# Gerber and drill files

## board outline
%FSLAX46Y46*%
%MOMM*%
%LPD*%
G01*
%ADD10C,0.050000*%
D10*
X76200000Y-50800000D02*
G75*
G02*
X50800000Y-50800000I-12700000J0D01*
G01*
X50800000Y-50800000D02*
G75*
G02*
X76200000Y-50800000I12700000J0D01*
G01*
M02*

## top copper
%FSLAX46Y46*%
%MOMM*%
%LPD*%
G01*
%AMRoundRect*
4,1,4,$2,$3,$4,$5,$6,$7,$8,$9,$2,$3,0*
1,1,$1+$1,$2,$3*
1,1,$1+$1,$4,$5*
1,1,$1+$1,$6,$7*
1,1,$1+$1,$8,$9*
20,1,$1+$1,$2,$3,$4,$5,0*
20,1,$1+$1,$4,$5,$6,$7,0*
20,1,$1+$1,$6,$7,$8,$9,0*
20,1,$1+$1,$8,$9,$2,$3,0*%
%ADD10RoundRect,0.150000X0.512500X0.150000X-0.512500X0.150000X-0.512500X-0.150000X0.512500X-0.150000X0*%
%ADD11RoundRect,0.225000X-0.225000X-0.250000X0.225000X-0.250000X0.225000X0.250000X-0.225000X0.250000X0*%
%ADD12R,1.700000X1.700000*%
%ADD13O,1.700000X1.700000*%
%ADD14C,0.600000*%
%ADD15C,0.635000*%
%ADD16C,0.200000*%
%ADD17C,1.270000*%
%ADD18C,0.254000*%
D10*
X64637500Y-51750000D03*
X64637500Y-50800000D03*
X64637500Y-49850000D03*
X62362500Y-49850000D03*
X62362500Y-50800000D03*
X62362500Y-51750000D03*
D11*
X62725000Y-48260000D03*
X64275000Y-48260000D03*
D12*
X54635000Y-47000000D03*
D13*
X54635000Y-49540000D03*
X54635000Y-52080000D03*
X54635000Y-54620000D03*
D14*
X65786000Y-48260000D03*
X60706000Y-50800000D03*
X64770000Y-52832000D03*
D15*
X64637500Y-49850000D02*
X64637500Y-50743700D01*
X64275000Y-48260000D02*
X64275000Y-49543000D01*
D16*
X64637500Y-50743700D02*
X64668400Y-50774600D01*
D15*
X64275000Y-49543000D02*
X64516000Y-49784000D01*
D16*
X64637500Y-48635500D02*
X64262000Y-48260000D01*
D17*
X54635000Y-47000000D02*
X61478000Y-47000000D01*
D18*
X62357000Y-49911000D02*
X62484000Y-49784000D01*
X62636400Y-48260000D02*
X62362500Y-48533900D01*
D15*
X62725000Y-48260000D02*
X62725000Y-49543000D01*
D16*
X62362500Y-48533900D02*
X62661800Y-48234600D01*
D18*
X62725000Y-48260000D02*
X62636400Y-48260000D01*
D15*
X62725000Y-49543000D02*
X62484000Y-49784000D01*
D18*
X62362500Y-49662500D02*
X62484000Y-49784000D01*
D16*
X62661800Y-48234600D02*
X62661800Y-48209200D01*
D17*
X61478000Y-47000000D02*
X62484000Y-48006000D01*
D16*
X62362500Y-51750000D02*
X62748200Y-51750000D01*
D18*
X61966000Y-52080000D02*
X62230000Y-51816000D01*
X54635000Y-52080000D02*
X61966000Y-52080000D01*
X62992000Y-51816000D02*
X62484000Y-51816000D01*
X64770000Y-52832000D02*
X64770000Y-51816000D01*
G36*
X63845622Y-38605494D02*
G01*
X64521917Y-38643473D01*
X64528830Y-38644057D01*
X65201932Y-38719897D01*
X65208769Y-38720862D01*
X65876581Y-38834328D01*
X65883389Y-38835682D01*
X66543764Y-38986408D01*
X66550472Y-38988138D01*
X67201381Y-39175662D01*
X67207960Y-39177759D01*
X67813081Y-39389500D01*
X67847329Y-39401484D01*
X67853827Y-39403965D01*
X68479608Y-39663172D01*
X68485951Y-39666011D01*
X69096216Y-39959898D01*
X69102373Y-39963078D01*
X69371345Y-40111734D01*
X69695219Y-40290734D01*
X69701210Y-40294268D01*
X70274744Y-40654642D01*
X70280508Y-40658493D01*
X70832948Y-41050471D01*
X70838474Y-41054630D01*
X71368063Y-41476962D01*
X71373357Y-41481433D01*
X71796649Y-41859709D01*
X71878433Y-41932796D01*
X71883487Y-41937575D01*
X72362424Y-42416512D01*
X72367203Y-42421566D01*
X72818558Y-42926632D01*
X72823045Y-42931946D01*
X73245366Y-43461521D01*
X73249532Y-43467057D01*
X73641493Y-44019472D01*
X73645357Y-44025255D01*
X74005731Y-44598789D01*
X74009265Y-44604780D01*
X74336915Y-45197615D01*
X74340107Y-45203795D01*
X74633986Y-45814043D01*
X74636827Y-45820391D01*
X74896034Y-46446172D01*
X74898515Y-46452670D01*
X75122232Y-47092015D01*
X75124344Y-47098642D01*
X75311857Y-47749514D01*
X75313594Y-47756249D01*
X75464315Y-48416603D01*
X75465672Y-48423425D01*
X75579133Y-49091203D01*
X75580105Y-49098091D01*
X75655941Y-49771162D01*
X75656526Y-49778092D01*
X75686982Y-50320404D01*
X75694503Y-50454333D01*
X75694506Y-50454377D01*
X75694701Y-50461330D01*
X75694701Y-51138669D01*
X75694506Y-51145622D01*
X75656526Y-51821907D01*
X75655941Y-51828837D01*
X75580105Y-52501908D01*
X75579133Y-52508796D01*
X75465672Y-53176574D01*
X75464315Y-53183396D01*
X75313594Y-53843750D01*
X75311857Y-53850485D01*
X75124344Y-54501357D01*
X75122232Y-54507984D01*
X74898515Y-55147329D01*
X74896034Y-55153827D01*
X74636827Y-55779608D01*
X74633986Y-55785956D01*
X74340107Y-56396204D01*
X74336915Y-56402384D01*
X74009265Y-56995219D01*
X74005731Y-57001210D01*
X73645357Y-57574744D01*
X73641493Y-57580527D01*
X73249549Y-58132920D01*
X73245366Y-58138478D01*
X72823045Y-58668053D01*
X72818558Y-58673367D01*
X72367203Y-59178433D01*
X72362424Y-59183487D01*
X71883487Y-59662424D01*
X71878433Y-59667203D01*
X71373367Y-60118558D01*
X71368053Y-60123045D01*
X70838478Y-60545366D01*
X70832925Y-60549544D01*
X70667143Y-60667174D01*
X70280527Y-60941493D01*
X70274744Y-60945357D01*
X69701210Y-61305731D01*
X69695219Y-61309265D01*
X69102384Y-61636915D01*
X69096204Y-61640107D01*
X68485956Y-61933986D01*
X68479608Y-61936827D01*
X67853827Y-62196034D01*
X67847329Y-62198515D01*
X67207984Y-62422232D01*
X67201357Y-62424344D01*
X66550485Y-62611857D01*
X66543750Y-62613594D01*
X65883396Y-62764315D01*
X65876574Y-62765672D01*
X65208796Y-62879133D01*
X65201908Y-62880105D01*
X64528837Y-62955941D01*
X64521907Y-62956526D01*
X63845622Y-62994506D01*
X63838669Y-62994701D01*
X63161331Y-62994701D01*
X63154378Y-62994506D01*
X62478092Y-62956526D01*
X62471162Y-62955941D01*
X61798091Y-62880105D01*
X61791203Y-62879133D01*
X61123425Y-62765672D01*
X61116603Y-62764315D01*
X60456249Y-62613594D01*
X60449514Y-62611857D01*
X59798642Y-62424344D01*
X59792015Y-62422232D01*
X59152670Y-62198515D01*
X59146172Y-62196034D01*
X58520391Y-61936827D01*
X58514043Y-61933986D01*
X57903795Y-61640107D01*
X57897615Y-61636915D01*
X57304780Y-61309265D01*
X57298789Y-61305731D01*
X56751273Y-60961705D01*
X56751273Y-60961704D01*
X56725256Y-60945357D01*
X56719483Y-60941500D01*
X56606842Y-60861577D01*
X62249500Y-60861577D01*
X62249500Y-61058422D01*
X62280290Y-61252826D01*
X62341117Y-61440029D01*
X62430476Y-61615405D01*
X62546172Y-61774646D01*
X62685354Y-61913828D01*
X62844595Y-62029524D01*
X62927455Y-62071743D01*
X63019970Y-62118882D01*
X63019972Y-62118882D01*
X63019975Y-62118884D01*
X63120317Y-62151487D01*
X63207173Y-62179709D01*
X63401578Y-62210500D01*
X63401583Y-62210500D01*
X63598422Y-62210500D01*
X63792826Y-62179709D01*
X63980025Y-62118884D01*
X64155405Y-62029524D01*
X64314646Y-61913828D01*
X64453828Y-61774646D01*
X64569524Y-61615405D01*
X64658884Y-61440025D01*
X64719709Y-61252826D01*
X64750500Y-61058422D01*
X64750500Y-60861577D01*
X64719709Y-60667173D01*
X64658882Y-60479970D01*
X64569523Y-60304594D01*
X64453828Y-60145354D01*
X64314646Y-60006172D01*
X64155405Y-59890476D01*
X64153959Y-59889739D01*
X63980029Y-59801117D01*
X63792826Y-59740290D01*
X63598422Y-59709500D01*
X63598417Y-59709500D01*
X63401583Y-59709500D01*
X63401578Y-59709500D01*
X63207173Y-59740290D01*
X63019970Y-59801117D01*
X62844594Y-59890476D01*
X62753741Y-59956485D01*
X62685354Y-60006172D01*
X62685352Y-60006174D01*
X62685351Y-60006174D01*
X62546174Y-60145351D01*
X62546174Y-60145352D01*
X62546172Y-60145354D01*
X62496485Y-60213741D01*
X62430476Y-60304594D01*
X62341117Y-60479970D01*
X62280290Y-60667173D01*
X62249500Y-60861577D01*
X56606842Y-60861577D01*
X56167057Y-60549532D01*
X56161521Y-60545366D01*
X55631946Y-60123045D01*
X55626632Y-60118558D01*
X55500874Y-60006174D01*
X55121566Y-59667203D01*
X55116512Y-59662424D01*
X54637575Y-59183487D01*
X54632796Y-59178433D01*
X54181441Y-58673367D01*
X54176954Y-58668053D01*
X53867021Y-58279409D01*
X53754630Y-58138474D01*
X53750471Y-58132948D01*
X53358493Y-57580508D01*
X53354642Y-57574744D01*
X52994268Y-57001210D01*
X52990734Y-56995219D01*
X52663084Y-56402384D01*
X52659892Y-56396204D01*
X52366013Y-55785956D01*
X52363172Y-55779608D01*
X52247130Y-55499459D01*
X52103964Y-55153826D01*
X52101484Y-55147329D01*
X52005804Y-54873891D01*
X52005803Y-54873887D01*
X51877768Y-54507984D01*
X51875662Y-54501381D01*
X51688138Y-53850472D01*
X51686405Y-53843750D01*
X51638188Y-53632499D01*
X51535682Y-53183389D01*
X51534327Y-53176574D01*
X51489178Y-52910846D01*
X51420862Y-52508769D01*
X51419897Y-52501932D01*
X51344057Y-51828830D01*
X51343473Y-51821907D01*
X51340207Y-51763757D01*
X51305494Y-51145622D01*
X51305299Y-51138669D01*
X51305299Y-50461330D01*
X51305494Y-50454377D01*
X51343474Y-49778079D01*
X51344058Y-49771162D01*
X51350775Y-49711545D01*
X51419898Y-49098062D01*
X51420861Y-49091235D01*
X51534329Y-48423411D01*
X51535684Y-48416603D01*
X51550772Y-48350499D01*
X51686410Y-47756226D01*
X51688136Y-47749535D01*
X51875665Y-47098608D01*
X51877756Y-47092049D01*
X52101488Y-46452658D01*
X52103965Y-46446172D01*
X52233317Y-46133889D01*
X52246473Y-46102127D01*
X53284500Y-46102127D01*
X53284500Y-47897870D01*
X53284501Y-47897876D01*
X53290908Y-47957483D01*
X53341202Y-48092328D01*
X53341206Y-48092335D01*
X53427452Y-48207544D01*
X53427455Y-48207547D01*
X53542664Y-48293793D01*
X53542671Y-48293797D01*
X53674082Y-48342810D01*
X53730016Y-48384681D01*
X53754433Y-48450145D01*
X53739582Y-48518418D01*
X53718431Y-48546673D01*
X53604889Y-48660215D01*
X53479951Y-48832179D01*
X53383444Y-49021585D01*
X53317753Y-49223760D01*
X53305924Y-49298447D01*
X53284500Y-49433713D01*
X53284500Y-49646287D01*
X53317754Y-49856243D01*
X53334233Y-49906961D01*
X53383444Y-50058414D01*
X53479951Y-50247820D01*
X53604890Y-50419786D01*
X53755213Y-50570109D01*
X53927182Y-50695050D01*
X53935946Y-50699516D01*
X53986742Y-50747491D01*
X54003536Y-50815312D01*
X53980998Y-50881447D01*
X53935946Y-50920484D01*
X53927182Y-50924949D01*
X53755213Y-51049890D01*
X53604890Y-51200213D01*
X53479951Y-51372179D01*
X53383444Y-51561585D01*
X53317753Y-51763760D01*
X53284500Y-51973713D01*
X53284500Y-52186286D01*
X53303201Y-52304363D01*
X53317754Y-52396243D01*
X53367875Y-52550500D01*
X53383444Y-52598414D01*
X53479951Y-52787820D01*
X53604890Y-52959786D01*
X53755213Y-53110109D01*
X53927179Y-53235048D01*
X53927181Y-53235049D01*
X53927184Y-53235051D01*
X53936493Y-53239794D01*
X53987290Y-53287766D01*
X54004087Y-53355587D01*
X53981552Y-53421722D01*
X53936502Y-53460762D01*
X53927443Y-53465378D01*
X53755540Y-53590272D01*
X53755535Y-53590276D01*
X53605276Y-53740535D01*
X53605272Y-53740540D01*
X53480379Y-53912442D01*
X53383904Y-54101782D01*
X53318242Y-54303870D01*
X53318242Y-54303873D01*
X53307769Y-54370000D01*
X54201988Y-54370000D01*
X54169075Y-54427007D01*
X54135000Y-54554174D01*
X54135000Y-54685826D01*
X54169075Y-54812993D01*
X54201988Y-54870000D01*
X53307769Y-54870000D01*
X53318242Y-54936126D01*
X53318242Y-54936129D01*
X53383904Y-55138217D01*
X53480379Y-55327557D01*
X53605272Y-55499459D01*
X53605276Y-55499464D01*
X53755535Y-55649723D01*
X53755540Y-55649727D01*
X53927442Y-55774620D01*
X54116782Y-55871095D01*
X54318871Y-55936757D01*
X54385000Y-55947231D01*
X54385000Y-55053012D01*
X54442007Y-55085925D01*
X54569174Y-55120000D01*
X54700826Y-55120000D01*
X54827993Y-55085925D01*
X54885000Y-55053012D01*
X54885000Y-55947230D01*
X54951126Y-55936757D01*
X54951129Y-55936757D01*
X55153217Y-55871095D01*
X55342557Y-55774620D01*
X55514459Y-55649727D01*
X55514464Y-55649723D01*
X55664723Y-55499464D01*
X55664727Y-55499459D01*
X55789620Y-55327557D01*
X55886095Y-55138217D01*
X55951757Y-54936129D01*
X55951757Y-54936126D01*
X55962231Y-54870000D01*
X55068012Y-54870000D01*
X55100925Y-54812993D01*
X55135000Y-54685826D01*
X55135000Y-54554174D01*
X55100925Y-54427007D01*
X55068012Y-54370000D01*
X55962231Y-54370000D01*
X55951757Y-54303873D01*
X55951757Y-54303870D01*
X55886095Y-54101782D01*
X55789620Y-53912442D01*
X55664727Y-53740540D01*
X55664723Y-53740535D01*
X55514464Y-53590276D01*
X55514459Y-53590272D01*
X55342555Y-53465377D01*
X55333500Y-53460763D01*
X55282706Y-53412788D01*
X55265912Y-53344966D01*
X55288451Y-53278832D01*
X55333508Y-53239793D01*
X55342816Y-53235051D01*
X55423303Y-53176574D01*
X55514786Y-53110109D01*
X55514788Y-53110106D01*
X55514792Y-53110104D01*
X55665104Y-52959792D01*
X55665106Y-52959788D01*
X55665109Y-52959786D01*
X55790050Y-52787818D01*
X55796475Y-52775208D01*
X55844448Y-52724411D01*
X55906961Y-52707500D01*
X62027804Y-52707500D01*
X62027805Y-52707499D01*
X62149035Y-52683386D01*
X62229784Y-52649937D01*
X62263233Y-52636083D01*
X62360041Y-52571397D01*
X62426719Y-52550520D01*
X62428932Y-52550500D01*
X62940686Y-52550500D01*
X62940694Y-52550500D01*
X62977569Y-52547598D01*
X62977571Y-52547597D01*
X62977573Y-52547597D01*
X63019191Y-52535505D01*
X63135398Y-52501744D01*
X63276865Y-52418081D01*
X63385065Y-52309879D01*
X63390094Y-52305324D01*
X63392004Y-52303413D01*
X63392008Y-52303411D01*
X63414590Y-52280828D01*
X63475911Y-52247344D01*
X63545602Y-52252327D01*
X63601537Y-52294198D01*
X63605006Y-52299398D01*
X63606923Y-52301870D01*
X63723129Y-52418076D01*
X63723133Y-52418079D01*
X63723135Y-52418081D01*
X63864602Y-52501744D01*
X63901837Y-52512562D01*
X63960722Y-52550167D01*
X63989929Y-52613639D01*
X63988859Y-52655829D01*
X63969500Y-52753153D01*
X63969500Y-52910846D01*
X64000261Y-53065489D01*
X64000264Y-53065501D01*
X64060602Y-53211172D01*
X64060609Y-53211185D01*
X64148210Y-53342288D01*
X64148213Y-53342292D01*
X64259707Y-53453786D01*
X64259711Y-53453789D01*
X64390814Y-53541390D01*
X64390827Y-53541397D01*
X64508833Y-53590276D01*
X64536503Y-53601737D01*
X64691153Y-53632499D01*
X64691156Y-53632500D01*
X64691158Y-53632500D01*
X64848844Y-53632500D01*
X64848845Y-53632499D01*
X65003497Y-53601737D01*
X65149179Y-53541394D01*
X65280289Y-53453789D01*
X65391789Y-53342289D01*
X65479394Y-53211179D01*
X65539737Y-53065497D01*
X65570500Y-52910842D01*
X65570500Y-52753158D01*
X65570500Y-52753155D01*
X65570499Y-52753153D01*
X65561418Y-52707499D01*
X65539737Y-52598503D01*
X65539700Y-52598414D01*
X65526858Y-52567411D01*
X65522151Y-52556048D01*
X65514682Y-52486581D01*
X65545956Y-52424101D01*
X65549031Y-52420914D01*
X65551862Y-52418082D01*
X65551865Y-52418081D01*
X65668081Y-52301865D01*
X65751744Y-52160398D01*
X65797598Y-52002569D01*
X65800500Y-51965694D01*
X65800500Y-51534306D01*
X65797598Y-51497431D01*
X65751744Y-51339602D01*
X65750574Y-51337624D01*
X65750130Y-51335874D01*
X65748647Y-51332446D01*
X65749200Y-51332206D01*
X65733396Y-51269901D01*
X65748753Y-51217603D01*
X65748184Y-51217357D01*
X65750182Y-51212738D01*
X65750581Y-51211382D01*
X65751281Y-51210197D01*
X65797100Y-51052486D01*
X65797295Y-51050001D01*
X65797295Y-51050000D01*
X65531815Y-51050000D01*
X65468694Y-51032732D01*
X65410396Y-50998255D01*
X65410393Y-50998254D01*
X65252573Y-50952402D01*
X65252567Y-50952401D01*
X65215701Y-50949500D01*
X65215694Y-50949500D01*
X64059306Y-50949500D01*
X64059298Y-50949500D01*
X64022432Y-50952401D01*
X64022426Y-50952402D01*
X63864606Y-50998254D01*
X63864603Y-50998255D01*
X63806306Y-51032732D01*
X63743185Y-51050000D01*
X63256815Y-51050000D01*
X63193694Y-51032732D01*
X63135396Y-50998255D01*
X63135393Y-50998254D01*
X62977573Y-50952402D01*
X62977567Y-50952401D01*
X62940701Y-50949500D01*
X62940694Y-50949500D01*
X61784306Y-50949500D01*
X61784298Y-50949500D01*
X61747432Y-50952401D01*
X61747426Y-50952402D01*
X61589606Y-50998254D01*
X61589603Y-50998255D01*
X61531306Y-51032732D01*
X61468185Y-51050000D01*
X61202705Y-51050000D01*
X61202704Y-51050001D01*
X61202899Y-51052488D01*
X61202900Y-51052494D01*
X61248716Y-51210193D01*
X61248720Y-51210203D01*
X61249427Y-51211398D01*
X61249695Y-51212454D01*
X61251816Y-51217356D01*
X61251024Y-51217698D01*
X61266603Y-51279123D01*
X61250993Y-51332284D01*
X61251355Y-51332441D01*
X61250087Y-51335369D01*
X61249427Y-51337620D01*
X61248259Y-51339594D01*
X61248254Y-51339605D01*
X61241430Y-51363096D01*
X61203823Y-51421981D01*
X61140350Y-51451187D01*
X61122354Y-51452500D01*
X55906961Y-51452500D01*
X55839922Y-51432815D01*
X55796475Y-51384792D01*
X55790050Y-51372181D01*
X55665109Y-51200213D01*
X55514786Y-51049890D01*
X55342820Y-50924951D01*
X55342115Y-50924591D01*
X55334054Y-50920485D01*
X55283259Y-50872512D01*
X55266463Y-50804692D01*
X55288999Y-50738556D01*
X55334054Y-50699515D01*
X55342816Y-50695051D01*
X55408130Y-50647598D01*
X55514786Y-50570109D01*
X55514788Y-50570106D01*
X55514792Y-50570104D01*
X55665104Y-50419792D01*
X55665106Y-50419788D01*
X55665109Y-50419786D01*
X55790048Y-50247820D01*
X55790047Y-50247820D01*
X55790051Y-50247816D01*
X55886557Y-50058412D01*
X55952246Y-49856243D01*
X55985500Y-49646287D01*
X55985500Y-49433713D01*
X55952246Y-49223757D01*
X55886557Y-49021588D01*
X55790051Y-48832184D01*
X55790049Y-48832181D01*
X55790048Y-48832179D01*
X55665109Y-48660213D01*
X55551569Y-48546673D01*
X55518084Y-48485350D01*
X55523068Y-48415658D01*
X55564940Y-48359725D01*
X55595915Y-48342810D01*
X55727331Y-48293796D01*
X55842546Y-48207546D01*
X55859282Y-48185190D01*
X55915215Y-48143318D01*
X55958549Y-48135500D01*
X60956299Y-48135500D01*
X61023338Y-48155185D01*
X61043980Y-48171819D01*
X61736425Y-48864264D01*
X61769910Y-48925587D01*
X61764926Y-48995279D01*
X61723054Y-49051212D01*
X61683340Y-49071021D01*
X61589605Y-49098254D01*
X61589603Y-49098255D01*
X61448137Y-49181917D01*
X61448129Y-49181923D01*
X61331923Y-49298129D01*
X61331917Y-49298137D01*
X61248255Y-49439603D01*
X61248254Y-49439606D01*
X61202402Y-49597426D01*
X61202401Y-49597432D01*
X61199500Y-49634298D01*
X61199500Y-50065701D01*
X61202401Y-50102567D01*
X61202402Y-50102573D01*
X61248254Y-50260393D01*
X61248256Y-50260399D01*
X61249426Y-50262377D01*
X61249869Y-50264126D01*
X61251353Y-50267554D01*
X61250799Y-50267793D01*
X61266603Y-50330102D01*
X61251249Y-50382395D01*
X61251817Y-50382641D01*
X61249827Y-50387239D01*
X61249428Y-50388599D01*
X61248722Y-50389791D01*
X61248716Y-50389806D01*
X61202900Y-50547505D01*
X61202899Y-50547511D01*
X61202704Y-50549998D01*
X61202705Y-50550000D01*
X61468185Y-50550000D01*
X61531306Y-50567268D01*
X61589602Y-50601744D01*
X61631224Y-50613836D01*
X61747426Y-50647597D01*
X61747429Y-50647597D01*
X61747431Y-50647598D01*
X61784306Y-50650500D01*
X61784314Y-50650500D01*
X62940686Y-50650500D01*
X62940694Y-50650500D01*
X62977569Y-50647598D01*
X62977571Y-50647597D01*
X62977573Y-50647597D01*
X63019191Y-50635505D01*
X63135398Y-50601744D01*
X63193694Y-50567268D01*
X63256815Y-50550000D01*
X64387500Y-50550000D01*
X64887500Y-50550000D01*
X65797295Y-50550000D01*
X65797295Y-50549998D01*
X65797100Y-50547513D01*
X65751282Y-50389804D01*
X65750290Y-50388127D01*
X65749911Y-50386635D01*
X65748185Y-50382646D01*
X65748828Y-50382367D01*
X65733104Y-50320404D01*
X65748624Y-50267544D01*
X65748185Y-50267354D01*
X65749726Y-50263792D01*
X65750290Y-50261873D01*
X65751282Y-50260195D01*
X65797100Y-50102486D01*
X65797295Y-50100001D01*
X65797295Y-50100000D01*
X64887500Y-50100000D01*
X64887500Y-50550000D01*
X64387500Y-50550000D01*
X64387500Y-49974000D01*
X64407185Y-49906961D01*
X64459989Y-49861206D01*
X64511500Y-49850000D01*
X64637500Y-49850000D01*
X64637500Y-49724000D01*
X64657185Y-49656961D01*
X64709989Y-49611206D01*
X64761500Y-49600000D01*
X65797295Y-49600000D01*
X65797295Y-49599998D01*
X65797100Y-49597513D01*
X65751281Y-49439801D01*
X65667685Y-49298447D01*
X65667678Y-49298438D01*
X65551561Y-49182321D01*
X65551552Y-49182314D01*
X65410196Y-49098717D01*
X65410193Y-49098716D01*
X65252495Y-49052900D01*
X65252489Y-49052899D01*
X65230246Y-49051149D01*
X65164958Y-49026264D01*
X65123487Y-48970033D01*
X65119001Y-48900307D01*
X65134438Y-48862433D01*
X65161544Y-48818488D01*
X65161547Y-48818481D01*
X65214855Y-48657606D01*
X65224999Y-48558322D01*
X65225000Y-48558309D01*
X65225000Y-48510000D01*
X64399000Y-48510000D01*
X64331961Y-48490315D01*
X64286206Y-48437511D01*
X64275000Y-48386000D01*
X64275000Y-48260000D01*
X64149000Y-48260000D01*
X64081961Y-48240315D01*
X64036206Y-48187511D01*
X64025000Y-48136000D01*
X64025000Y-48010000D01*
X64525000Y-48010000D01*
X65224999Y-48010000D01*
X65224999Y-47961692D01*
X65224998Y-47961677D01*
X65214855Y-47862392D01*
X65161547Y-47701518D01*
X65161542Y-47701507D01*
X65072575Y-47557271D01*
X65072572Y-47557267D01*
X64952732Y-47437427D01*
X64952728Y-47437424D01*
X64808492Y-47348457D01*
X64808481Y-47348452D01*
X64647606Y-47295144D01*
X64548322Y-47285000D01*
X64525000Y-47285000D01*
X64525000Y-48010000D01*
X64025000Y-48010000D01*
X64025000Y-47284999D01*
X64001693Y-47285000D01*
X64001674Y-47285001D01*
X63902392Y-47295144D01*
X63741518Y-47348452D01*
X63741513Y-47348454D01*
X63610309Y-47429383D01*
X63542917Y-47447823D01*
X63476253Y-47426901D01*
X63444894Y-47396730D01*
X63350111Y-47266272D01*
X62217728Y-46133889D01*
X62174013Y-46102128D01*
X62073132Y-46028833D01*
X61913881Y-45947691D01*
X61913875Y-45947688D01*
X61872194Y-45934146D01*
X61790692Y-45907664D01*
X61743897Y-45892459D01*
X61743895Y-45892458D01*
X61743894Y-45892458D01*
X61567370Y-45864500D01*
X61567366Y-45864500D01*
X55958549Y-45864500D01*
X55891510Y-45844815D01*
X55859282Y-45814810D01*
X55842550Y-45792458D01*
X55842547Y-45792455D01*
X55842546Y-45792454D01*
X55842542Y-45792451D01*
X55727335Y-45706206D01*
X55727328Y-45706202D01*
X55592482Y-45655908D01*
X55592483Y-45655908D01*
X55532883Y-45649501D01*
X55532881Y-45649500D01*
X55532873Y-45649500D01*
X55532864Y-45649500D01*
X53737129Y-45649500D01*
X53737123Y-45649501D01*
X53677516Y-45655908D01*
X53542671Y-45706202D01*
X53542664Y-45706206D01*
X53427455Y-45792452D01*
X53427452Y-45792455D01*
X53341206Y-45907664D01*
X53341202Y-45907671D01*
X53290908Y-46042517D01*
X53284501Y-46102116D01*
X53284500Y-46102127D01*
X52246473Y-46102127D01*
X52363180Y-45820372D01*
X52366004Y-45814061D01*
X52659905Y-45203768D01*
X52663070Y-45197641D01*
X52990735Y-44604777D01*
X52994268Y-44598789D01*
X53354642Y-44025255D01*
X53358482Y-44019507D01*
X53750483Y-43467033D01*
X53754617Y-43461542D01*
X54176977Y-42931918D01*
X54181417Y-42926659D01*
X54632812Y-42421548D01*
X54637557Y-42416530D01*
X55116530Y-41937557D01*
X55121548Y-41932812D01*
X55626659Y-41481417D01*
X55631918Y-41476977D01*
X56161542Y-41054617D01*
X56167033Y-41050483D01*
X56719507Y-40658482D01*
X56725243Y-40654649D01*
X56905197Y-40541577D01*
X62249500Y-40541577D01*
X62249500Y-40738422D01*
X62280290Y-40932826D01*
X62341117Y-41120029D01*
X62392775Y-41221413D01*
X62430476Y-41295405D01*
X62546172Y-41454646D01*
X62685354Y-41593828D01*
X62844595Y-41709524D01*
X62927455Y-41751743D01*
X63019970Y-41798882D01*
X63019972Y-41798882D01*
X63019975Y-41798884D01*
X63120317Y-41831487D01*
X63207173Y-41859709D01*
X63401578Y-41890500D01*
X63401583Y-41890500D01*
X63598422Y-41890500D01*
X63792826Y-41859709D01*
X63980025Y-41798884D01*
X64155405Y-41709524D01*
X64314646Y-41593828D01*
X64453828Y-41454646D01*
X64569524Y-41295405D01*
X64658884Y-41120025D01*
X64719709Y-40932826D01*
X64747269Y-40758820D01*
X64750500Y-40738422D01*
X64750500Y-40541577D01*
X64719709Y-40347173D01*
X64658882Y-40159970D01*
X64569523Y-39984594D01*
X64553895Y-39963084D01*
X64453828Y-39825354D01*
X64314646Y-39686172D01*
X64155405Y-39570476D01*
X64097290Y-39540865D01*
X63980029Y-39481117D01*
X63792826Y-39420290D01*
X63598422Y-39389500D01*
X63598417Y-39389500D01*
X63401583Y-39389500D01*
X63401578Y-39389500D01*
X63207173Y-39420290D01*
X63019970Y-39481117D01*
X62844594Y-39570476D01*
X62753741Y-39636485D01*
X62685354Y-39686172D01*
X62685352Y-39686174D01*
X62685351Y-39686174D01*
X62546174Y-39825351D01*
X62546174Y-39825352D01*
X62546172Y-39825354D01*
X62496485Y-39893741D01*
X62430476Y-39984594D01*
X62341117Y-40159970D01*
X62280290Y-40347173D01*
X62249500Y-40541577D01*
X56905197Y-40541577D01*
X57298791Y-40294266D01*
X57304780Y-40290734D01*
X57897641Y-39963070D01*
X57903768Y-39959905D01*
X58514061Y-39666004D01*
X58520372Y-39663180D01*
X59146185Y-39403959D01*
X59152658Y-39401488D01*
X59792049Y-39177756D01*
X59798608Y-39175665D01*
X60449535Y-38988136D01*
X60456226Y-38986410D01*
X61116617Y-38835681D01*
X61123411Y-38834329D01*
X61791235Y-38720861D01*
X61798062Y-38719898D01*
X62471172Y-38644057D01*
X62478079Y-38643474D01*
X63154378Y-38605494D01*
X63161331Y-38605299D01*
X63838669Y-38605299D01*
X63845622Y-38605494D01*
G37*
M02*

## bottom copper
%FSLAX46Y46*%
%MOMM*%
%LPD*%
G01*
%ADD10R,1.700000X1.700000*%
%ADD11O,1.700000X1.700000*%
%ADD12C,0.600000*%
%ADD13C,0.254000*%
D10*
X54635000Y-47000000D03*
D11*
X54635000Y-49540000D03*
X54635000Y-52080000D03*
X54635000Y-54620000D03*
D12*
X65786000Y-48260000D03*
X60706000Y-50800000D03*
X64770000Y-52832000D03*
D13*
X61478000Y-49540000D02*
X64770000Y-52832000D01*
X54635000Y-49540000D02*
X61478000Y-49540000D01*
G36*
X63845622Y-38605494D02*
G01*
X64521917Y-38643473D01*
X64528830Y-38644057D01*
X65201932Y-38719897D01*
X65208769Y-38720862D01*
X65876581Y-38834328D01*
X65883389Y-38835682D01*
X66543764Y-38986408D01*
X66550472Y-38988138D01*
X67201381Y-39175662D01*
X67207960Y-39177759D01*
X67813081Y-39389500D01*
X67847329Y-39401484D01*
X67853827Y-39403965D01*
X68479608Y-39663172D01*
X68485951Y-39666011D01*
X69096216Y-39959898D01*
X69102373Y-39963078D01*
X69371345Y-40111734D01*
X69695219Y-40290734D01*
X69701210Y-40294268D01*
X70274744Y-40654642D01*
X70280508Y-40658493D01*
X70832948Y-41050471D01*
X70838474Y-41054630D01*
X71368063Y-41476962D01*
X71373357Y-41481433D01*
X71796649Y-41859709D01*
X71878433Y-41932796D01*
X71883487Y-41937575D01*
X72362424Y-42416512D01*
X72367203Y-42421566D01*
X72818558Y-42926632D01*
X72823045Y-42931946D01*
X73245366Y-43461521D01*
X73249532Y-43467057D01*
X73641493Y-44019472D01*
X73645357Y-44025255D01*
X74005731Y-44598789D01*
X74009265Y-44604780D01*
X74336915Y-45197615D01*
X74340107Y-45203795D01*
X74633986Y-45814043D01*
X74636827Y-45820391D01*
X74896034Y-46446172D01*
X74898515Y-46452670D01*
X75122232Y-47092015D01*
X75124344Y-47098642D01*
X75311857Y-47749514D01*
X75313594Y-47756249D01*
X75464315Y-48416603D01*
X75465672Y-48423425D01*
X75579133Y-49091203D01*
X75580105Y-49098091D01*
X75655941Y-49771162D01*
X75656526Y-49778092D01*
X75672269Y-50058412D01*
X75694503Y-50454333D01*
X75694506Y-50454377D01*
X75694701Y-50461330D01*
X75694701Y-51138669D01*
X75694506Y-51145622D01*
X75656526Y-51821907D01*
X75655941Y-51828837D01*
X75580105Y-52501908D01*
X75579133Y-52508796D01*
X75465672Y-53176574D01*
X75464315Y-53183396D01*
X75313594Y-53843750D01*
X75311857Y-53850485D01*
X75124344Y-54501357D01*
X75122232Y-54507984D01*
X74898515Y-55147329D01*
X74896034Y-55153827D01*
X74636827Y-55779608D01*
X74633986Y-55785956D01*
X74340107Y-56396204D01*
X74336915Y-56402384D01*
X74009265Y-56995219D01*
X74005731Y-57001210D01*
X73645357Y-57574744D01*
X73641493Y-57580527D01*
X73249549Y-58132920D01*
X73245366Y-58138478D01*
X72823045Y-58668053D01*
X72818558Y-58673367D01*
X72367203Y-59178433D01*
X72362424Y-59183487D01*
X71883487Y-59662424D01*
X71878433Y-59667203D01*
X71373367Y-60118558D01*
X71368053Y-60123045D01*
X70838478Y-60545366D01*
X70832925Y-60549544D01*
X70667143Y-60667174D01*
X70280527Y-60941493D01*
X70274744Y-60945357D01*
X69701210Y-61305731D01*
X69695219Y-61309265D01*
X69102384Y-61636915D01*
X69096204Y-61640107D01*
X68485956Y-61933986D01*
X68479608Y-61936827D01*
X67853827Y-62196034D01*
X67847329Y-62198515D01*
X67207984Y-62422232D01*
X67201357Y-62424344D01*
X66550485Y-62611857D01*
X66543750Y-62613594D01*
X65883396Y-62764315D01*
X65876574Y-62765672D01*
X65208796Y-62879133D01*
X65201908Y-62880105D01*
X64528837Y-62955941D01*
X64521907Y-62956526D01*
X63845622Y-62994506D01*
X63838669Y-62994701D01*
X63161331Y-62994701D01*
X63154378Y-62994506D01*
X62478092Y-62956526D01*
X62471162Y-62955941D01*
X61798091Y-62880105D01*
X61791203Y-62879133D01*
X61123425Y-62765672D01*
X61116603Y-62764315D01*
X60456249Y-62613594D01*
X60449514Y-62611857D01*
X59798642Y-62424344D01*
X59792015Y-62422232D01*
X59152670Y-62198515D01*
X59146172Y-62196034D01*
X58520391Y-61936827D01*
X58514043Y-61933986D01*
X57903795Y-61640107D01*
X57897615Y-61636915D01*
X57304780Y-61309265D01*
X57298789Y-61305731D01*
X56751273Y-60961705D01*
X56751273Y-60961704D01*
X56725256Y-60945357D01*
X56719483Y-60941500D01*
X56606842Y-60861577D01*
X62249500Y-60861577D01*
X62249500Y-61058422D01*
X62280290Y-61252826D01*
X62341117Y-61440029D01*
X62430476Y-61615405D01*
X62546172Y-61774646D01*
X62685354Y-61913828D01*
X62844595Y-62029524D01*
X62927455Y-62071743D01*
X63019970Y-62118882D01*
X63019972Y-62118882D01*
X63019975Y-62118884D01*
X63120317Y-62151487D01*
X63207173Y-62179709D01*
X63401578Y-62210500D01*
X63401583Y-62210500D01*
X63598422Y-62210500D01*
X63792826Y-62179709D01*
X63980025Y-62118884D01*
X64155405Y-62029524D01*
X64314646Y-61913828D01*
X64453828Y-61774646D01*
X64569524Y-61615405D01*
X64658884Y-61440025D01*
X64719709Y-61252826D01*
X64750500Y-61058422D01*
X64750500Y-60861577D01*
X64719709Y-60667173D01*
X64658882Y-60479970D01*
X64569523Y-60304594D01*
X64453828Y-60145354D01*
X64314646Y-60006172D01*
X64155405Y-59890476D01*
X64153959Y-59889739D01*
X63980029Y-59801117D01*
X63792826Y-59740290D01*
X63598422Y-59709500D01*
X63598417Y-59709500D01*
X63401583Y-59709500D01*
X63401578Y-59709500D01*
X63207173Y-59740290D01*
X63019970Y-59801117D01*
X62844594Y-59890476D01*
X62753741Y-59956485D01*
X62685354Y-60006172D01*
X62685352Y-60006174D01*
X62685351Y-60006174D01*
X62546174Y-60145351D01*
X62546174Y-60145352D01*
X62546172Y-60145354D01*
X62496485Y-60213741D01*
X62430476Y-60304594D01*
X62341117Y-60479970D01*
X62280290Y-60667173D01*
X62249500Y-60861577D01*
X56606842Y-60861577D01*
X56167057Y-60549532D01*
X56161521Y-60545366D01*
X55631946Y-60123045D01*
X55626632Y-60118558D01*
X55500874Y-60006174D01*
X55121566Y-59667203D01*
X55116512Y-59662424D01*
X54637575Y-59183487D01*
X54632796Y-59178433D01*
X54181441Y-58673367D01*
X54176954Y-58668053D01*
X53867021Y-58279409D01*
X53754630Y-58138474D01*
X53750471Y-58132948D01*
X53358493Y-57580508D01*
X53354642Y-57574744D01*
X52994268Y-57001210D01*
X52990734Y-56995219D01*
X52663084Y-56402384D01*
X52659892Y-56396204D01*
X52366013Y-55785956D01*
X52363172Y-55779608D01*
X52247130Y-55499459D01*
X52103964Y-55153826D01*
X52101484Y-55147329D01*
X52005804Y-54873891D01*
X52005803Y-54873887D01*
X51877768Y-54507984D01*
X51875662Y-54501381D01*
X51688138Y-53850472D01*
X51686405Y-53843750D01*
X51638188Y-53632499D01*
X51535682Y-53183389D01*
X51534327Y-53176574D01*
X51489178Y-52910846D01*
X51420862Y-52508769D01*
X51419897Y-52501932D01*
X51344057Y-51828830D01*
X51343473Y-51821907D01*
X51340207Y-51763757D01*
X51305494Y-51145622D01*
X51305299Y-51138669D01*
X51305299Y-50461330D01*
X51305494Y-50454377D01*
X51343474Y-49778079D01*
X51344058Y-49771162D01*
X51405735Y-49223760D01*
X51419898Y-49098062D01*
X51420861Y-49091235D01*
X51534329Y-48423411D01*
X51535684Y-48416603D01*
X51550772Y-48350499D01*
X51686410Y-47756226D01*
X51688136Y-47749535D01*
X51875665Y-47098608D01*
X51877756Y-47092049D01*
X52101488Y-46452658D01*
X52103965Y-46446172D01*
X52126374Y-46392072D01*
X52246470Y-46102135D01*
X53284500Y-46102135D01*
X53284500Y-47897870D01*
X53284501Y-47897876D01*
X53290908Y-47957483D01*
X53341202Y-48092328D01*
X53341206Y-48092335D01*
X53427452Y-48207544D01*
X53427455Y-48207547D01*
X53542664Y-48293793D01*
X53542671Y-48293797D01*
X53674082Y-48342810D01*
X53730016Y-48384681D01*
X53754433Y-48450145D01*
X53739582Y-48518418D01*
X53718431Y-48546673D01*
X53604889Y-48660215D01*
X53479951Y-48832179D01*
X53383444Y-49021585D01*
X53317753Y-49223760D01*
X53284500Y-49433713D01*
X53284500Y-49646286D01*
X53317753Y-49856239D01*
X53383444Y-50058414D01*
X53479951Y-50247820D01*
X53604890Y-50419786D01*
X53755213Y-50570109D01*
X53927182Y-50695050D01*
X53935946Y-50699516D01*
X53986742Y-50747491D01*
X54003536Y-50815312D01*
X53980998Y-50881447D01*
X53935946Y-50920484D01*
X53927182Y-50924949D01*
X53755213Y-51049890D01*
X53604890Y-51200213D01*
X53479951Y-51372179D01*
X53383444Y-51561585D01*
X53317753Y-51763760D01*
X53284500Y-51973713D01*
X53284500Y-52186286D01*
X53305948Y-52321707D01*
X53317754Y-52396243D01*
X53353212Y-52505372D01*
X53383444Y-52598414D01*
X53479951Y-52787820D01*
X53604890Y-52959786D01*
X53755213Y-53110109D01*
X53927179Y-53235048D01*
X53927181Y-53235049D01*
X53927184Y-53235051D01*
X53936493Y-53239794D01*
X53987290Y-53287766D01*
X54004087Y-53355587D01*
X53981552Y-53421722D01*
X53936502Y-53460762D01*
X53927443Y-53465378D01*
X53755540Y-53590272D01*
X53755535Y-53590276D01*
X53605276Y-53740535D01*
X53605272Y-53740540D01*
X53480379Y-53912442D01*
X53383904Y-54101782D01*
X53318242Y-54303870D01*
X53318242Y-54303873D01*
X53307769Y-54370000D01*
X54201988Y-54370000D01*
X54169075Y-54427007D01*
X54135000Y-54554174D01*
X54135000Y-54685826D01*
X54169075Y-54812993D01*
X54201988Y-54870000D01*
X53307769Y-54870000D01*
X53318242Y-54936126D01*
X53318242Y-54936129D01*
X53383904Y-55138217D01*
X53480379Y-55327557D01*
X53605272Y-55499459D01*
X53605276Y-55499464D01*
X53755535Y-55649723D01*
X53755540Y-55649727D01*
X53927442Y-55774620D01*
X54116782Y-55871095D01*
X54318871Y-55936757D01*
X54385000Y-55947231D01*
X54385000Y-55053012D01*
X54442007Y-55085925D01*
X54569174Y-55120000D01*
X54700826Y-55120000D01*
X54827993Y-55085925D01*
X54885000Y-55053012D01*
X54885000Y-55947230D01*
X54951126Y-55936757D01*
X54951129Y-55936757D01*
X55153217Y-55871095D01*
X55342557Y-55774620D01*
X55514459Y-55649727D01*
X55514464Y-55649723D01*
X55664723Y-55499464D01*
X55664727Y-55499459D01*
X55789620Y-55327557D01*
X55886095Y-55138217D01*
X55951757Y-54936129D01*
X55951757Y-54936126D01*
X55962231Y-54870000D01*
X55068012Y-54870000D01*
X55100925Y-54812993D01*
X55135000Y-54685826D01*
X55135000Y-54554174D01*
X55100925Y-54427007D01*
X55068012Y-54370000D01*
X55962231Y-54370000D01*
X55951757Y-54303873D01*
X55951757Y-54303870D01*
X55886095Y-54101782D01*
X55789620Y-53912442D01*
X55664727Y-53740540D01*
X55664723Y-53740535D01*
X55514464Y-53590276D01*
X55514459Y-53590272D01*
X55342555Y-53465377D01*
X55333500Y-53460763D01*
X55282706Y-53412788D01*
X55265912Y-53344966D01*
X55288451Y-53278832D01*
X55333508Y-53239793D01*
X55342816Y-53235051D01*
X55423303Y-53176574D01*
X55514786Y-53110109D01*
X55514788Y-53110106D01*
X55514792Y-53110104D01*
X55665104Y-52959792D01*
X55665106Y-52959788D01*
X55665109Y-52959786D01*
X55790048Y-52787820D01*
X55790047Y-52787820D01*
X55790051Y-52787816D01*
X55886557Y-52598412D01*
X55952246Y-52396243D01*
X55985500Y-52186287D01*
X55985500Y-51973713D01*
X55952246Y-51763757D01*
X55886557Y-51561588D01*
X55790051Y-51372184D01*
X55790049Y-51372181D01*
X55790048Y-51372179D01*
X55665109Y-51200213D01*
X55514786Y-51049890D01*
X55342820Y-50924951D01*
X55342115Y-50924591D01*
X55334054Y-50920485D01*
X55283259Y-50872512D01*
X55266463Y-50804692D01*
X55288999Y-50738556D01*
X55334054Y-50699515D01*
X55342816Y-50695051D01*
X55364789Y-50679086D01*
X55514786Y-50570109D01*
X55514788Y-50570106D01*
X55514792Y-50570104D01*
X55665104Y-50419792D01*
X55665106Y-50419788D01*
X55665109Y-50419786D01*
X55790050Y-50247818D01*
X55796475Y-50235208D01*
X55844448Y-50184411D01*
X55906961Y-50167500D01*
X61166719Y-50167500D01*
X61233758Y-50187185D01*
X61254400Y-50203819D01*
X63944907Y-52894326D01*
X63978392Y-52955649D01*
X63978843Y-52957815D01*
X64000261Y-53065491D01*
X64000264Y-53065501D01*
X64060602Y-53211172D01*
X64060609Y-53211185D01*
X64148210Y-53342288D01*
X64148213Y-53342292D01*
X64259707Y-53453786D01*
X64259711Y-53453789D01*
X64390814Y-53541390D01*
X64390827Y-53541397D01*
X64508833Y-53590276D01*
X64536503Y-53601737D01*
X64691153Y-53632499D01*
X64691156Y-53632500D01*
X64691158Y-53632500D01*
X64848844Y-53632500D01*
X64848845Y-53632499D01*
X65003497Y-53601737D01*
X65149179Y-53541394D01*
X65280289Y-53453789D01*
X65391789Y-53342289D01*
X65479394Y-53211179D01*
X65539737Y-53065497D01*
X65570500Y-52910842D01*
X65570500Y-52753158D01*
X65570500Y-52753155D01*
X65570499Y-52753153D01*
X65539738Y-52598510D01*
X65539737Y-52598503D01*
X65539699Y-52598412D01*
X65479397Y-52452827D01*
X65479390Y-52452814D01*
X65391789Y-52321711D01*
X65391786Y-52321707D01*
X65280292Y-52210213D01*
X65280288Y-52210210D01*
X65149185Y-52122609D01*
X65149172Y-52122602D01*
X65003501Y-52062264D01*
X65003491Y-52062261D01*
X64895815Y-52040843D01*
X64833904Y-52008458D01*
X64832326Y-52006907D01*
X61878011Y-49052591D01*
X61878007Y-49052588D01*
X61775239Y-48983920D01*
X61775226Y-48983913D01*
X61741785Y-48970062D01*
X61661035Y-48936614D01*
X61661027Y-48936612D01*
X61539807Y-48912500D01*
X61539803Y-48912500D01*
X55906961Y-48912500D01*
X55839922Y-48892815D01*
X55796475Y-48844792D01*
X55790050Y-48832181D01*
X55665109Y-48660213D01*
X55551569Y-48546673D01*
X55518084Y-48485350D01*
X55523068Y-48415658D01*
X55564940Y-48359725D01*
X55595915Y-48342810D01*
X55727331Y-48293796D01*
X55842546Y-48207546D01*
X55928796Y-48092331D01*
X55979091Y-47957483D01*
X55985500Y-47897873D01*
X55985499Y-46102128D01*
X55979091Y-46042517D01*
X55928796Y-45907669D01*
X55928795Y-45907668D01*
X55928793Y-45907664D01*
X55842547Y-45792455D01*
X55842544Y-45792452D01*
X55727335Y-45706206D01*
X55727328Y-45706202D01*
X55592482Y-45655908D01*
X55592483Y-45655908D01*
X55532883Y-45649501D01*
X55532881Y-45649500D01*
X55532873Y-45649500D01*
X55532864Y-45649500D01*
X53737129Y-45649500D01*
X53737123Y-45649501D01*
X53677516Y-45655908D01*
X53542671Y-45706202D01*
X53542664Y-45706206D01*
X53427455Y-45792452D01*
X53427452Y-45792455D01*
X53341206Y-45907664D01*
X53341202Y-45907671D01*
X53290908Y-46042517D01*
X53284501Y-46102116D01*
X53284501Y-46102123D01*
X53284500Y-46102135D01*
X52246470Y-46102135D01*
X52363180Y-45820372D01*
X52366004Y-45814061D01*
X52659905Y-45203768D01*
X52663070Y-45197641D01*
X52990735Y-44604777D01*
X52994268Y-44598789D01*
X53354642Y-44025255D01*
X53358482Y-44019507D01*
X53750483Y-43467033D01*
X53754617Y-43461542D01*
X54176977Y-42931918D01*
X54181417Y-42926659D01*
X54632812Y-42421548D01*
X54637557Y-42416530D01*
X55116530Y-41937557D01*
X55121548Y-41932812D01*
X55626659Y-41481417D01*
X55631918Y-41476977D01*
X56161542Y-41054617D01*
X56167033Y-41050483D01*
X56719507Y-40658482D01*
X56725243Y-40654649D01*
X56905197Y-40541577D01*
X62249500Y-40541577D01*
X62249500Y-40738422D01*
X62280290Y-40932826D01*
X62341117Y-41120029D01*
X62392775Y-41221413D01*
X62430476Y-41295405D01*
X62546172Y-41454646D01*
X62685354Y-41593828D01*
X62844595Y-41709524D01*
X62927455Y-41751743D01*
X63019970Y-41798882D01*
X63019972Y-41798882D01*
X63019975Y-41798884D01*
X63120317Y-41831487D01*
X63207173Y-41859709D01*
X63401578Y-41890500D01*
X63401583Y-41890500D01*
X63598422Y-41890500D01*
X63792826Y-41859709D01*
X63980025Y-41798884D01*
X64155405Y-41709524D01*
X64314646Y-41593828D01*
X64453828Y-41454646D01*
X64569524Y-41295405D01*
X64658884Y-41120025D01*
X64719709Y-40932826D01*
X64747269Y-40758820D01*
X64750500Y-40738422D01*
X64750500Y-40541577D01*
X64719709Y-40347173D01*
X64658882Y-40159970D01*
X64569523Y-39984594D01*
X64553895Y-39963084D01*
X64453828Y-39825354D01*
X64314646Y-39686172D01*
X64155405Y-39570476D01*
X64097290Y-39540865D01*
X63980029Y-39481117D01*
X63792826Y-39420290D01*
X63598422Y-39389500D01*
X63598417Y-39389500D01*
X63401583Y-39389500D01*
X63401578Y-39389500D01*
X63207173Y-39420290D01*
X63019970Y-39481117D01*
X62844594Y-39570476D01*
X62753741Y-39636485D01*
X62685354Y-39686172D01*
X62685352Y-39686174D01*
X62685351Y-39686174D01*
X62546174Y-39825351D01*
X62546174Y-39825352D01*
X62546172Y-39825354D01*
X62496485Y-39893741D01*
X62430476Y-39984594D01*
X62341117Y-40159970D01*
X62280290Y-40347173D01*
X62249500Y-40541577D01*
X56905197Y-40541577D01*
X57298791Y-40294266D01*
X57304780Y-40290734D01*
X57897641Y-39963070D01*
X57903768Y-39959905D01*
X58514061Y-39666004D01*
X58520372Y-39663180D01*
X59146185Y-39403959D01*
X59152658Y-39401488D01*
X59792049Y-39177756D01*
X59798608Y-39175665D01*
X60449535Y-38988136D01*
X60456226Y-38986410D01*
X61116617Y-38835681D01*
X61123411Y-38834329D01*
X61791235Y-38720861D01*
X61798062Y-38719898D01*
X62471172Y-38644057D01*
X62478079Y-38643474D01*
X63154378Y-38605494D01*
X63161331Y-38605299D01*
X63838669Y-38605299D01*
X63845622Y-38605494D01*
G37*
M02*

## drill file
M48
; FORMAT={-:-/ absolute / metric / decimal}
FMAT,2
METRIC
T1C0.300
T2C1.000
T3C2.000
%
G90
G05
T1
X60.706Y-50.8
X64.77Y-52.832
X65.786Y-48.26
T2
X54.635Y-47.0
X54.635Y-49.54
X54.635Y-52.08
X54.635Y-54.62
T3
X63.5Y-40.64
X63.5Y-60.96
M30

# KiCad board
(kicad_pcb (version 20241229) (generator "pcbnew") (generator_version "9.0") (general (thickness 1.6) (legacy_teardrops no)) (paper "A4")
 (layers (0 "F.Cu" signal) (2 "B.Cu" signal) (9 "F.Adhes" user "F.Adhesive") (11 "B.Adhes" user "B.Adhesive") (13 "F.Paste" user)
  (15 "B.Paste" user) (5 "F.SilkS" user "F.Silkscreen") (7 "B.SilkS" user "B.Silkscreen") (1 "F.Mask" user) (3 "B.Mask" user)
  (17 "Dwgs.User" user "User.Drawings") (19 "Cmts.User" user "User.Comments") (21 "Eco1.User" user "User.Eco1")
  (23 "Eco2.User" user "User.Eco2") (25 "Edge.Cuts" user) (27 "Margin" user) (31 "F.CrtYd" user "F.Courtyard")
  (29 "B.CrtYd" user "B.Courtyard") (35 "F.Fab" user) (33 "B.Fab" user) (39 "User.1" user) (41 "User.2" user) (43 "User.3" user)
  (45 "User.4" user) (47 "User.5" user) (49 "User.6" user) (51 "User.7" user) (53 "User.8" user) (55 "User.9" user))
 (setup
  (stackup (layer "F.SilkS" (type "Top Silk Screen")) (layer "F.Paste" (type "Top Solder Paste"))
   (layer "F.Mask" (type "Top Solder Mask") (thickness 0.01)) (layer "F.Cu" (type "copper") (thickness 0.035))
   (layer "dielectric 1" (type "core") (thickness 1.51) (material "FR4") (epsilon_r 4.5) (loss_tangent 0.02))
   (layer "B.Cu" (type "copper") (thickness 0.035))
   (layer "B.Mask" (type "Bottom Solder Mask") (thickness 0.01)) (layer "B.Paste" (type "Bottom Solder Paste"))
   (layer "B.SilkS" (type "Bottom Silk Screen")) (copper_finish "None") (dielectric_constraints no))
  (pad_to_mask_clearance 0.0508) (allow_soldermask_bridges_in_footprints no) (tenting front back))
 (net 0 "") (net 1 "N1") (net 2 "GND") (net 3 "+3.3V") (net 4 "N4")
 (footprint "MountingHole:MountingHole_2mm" (layer "F.Cu") (at 63.5 40.64)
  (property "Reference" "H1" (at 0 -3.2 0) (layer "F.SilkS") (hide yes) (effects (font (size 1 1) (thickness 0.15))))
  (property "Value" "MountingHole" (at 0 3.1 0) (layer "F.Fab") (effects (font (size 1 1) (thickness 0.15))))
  (pad "" np_thru_hole circle (at 0 0) (size 2 2) (drill 2) (layers "*.Cu" "*.Mask")))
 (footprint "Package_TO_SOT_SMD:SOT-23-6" (layer "F.Cu") (at 63.5 50.8 180)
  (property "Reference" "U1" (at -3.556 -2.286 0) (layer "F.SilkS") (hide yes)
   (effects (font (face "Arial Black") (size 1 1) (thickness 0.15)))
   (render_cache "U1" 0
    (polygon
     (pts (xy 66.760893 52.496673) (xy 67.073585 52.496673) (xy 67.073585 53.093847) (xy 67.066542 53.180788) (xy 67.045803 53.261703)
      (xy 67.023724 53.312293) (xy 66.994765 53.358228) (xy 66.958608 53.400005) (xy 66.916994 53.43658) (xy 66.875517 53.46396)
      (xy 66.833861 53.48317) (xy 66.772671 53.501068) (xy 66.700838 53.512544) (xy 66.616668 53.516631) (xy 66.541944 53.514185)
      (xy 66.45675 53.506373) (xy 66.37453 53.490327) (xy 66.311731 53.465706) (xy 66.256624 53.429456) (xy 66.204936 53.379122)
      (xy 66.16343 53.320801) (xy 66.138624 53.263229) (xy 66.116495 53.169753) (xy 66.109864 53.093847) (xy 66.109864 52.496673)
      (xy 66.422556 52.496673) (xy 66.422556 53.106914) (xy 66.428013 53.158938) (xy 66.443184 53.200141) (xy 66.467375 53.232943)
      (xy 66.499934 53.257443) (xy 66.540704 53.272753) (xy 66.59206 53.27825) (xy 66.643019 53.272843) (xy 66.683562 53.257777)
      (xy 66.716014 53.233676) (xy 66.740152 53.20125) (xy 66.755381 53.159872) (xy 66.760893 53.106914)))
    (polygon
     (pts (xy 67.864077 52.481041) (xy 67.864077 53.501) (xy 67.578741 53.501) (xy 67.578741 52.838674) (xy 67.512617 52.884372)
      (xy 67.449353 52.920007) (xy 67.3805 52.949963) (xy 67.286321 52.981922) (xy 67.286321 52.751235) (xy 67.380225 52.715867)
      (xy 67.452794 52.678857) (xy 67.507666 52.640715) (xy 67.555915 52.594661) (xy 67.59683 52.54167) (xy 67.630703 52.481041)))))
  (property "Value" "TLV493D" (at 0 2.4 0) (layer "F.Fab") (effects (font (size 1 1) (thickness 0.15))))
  (pad "1" smd roundrect (at -1.1375 -0.95 180) (size 1.325 0.6) (layers "F.Cu" "F.Mask" "F.Paste") (roundrect_rratio 0.25) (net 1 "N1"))
  (pad "2" smd roundrect (at -1.1375 0 180) (size 1.325 0.6) (layers "F.Cu" "F.Mask" "F.Paste") (roundrect_rratio 0.25) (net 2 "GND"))
  (pad "3" smd roundrect (at -1.1375 0.95 180) (size 1.325 0.6) (layers "F.Cu" "F.Mask" "F.Paste") (roundrect_rratio 0.25) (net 2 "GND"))
  (pad "4" smd roundrect (at 1.1375 0.95 180) (size 1.325 0.6) (layers "F.Cu" "F.Mask" "F.Paste") (roundrect_rratio 0.25) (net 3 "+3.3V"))
  (pad "5" smd roundrect (at 1.1375 0 180) (size 1.325 0.6) (layers "F.Cu" "F.Mask" "F.Paste") (roundrect_rratio 0.25) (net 2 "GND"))
  (pad "6" smd roundrect (at 1.1375 -0.95 180) (size 1.325 0.6) (layers "F.Cu" "F.Mask" "F.Paste") (roundrect_rratio 0.25) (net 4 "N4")))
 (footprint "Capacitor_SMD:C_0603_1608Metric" (layer "F.Cu") (at 63.5 48.26)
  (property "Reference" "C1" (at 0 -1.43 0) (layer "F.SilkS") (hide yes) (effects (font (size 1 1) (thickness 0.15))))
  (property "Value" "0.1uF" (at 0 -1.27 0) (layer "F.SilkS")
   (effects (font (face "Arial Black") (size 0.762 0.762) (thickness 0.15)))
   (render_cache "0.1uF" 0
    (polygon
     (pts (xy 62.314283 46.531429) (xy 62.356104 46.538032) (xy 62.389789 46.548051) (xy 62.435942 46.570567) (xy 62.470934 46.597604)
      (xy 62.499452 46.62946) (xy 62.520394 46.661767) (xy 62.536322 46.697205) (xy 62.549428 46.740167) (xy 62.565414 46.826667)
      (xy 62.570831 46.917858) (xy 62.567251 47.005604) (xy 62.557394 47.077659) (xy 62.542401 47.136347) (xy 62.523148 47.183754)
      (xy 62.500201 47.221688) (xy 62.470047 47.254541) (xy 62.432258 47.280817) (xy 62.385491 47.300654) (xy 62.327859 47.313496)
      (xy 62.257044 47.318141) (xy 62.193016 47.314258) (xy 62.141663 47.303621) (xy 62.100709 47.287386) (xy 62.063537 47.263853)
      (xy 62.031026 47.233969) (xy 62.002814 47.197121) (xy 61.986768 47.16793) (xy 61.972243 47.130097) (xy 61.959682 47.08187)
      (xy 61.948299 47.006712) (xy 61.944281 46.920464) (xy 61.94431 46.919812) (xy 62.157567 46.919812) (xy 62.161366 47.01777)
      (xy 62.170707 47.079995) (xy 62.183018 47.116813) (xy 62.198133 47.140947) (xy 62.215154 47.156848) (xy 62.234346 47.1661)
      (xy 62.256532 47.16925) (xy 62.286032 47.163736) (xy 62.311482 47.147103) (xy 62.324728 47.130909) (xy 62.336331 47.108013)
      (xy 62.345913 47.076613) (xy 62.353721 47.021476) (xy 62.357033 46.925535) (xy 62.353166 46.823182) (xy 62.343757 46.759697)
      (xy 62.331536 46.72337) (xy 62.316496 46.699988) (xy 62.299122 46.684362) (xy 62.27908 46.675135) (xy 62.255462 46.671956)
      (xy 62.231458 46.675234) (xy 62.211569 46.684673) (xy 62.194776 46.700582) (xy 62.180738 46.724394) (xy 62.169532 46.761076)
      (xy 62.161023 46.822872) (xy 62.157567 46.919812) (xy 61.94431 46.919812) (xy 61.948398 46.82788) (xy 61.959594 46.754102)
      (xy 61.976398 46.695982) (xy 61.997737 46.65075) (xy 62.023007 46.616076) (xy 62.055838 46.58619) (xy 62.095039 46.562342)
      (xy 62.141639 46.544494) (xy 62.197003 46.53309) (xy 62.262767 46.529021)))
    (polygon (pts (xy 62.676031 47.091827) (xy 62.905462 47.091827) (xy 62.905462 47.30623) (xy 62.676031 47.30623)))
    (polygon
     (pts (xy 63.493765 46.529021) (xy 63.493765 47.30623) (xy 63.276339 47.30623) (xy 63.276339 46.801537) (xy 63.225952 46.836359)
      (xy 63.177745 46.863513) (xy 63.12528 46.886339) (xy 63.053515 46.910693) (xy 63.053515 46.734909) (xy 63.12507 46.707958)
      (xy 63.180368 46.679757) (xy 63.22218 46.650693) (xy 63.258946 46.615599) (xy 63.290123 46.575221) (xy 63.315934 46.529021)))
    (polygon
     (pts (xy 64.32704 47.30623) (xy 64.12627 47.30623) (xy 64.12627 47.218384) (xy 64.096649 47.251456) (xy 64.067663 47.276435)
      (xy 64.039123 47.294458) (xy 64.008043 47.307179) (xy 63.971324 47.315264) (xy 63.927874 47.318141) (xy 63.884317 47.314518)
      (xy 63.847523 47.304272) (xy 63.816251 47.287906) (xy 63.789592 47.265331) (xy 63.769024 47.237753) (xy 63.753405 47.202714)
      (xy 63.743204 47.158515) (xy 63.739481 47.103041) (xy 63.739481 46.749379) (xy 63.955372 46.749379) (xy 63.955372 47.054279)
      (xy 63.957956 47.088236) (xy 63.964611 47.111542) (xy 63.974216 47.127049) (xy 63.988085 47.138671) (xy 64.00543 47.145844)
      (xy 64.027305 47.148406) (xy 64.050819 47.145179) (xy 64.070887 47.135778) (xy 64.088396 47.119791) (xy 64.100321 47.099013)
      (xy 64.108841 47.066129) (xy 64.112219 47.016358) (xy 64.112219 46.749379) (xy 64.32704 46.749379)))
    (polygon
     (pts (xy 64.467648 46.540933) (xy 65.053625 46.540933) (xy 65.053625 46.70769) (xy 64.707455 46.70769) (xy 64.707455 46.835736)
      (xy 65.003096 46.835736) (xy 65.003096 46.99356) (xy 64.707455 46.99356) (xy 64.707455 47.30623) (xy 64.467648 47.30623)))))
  (pad "1" smd roundrect (at -0.775 0) (size 0.9 0.95) (layers "F.Cu" "F.Mask" "F.Paste") (roundrect_rratio 0.25) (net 3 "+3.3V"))
  (pad "2" smd roundrect (at 0.775 0) (size 0.9 0.95) (layers "F.Cu" "F.Mask" "F.Paste") (roundrect_rratio 0.25) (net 2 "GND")))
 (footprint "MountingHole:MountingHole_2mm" (layer "F.Cu") (at 63.5 60.96)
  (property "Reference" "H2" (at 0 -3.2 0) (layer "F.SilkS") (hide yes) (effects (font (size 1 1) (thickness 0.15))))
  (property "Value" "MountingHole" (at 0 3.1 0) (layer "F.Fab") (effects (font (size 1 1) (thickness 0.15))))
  (pad "" np_thru_hole circle (at 0 0) (size 2 2) (drill 2) (layers "*.Cu" "*.Mask")))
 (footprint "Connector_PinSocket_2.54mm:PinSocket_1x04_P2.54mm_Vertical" (layer "B.Cu") (at 54.635 47 180)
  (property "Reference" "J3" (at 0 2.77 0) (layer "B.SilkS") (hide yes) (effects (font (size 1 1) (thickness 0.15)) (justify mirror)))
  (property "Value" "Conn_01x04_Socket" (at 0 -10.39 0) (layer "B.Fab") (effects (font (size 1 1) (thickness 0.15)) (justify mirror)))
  (pad "1" thru_hole rect (at 0 0 180) (size 1.7 1.7) (drill 1) (layers "*.Cu" "*.Mask") (remove_unused_layers no) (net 3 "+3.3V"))
  (pad "2" thru_hole oval (at 0 -2.54 180) (size 1.7 1.7) (drill 1) (layers "*.Cu" "*.Mask") (remove_unused_layers no) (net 1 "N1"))
  (pad "3" thru_hole oval (at 0 -5.08 180) (size 1.7 1.7) (drill 1) (layers "*.Cu" "*.Mask") (remove_unused_layers no) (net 4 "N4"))
  (pad "4" thru_hole oval (at 0 -7.62 180) (size 1.7 1.7) (drill 1) (layers "*.Cu" "*.Mask") (remove_unused_layers no) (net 2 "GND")))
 (gr_circle (center 63.5 50.8) (end 76.2 50.8) (stroke (width 0.05) (type default)) (fill no) (layer "Edge.Cuts"))
 (segment (start 64.6375 49.85) (end 64.6375 50.7437) (width 0.635) (layer "F.Cu") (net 2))
 (segment (start 64.275 48.26) (end 64.275 49.543) (width 0.635) (layer "F.Cu") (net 2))
 (segment (start 64.6375 50.7437) (end 64.6684 50.7746) (width 0.2) (layer "F.Cu") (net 2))
 (segment (start 64.275 49.543) (end 64.516 49.784) (width 0.635) (layer "F.Cu") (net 2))
 (segment (start 64.6375 48.6355) (end 64.262 48.26) (width 0.2) (layer "F.Cu") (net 2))
 (via (at 65.786 48.26) (size 0.6) (drill 0.3) (layers "F.Cu" "B.Cu") (free yes) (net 2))
 (via (at 60.706 50.8) (size 0.6) (drill 0.3) (layers "F.Cu" "B.Cu") (free yes) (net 2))
 (segment (start 54.635 47) (end 61.478 47) (width 1.27) (layer "F.Cu") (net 3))
 (segment (start 62.357 49.911) (end 62.484 49.784) (width 0.254) (layer "F.Cu") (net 3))
 (segment (start 62.6364 48.26) (end 62.3625 48.5339) (width 0.254) (layer "F.Cu") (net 3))
 (segment (start 62.725 48.26) (end 62.725 49.543) (width 0.635) (layer "F.Cu") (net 3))
 (segment (start 62.3625 48.5339) (end 62.6618 48.2346) (width 0.2) (layer "F.Cu") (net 3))
 (segment (start 62.725 48.26) (end 62.6364 48.26) (width 0.254) (layer "F.Cu") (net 3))
 (segment (start 62.725 49.543) (end 62.484 49.784) (width 0.635) (layer "F.Cu") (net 3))
 (segment (start 62.3625 49.6625) (end 62.484 49.784) (width 0.254) (layer "F.Cu") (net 3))
 (segment (start 62.6618 48.2346) (end 62.6618 48.2092) (width 0.2) (layer "F.Cu") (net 3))
 (segment (start 61.478 47) (end 62.484 48.006) (width 1.27) (layer "F.Cu") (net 3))
 (segment (start 62.3625 51.75) (end 62.7482 51.75) (width 0.2) (layer "F.Cu") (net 4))
 (segment (start 61.966 52.08) (end 62.23 51.816) (width 0.254) (layer "F.Cu") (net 4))
 (segment (start 54.635 52.08) (end 61.966 52.08) (width 0.254) (layer "F.Cu") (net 4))
 (segment (start 62.992 51.816) (end 62.484 51.816) (width 0.254) (layer "F.Cu") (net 4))
 (segment (start 64.77 52.832) (end 64.77 51.816) (width 0.254) (layer "F.Cu") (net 1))
 (via (at 64.77 52.832) (size 0.6) (drill 0.3) (layers "F.Cu" "B.Cu") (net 1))
 (segment (start 61.478 49.54) (end 64.77 52.832) (width 0.254) (layer "B.Cu") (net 1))
 (segment (start 54.635 49.54) (end 61.478 49.54) (width 0.254) (layer "B.Cu") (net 1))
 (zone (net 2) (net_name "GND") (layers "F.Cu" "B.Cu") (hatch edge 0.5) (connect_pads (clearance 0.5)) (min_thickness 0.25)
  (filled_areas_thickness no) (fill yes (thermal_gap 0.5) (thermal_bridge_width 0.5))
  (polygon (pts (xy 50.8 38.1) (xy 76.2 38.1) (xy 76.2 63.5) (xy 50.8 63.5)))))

